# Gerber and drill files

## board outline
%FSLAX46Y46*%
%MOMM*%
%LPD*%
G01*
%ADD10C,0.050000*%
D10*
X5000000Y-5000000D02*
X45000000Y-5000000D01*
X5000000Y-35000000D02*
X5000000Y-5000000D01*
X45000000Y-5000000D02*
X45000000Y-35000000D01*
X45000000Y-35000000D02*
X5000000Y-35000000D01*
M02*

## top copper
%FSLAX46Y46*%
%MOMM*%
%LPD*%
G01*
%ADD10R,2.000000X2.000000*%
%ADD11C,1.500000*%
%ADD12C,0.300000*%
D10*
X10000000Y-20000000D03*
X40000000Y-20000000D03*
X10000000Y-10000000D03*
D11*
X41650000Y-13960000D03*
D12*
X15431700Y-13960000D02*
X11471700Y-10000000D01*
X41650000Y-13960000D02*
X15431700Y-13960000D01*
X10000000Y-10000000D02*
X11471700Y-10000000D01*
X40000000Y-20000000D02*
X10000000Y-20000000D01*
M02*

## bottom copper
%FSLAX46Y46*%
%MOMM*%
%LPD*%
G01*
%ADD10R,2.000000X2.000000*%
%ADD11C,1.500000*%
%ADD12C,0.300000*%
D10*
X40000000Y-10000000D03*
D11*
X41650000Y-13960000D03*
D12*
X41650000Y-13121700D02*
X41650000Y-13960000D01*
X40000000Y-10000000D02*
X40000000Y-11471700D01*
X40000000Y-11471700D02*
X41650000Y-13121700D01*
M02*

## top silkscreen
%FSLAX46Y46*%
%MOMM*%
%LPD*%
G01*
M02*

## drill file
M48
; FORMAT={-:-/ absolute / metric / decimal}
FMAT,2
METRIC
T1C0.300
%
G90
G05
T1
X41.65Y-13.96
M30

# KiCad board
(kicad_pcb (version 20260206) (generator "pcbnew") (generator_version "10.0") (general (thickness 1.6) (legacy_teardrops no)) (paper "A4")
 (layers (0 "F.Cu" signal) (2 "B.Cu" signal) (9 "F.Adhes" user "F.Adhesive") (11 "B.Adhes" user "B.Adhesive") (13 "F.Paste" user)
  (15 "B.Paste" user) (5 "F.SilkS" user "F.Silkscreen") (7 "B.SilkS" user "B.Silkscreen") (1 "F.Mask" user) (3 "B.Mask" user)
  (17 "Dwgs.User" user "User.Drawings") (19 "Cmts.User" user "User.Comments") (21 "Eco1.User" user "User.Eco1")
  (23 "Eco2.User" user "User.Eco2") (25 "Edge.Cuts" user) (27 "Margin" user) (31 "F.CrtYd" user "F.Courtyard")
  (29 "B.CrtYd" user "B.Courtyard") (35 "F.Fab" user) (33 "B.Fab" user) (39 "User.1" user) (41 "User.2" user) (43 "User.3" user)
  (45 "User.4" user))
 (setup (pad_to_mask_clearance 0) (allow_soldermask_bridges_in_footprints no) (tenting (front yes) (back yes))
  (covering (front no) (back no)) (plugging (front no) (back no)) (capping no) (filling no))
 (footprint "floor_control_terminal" (layer "F.Cu") (at 10 20)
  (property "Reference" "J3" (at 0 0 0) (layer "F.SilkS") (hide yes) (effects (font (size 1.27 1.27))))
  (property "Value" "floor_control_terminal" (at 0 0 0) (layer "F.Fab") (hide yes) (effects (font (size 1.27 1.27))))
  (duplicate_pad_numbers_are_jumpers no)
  (pad "1" smd rect (at 0 0) (size 2 2) (layers "F.Cu" "F.Mask" "F.Paste") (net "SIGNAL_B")))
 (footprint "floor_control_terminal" (layer "F.Cu") (at 40 20)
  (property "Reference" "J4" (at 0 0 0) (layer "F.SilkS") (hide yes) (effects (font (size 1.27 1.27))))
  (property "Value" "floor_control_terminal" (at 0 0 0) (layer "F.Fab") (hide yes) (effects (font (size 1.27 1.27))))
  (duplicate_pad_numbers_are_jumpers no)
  (pad "1" smd rect (at 0 0) (size 2 2) (layers "F.Cu" "F.Mask" "F.Paste") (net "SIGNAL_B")))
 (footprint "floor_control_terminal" (layer "F.Cu") (at 10 10)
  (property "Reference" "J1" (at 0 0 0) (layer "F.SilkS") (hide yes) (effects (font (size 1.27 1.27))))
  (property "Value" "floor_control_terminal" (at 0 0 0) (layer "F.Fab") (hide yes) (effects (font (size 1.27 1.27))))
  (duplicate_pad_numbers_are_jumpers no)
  (pad "1" smd rect (at 0 0) (size 2 2) (layers "F.Cu" "F.Mask" "F.Paste") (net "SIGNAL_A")))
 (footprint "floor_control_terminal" (layer "B.Cu") (at 40 10)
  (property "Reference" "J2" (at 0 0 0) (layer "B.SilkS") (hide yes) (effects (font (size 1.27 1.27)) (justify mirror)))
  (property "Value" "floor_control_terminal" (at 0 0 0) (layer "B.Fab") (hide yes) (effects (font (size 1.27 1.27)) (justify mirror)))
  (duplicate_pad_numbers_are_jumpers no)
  (pad "1" smd rect (at 0 0) (size 2 2) (layers "B.Cu" "B.Mask" "B.Paste") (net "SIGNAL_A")))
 (gr_line (start 5 5) (end 45 5) (stroke (width 0.05) (type default)) (layer "Edge.Cuts"))
 (gr_line (start 5 35) (end 5 5) (stroke (width 0.05) (type default)) (layer "Edge.Cuts"))
 (gr_line (start 45 5) (end 45 35) (stroke (width 0.05) (type default)) (layer "Edge.Cuts"))
 (gr_line (start 45 35) (end 5 35) (stroke (width 0.05) (type default)) (layer "Edge.Cuts"))
 (segment (start 15.4317 13.96) (end 11.4717 10) (width 0.3) (layer "F.Cu") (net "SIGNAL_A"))
 (segment (start 41.65 13.96) (end 15.4317 13.96) (width 0.3) (layer "F.Cu") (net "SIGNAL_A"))
 (segment (start 10 10) (end 11.4717 10) (width 0.3) (layer "F.Cu") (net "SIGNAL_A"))
 (via (at 41.65 13.96) (size 1.5) (drill 0.3) (layers "F.Cu" "B.Cu") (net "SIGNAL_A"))
 (segment (start 41.65 13.1217) (end 41.65 13.96) (width 0.3) (layer "B.Cu") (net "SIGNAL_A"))
 (segment (start 40 10) (end 40 11.4717) (width 0.3) (layer "B.Cu") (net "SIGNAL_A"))
 (segment (start 40 11.4717) (end 41.65 13.1217) (width 0.3) (layer "B.Cu") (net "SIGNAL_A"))
 (segment (start 40 20) (end 10 20) (width 0.3) (layer "F.Cu") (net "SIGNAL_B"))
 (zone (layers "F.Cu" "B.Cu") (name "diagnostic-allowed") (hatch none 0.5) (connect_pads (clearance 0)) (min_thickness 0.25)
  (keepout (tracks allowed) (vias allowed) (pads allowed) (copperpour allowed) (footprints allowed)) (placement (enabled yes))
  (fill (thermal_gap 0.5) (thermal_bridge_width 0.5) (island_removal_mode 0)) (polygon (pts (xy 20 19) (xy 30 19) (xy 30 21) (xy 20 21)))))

